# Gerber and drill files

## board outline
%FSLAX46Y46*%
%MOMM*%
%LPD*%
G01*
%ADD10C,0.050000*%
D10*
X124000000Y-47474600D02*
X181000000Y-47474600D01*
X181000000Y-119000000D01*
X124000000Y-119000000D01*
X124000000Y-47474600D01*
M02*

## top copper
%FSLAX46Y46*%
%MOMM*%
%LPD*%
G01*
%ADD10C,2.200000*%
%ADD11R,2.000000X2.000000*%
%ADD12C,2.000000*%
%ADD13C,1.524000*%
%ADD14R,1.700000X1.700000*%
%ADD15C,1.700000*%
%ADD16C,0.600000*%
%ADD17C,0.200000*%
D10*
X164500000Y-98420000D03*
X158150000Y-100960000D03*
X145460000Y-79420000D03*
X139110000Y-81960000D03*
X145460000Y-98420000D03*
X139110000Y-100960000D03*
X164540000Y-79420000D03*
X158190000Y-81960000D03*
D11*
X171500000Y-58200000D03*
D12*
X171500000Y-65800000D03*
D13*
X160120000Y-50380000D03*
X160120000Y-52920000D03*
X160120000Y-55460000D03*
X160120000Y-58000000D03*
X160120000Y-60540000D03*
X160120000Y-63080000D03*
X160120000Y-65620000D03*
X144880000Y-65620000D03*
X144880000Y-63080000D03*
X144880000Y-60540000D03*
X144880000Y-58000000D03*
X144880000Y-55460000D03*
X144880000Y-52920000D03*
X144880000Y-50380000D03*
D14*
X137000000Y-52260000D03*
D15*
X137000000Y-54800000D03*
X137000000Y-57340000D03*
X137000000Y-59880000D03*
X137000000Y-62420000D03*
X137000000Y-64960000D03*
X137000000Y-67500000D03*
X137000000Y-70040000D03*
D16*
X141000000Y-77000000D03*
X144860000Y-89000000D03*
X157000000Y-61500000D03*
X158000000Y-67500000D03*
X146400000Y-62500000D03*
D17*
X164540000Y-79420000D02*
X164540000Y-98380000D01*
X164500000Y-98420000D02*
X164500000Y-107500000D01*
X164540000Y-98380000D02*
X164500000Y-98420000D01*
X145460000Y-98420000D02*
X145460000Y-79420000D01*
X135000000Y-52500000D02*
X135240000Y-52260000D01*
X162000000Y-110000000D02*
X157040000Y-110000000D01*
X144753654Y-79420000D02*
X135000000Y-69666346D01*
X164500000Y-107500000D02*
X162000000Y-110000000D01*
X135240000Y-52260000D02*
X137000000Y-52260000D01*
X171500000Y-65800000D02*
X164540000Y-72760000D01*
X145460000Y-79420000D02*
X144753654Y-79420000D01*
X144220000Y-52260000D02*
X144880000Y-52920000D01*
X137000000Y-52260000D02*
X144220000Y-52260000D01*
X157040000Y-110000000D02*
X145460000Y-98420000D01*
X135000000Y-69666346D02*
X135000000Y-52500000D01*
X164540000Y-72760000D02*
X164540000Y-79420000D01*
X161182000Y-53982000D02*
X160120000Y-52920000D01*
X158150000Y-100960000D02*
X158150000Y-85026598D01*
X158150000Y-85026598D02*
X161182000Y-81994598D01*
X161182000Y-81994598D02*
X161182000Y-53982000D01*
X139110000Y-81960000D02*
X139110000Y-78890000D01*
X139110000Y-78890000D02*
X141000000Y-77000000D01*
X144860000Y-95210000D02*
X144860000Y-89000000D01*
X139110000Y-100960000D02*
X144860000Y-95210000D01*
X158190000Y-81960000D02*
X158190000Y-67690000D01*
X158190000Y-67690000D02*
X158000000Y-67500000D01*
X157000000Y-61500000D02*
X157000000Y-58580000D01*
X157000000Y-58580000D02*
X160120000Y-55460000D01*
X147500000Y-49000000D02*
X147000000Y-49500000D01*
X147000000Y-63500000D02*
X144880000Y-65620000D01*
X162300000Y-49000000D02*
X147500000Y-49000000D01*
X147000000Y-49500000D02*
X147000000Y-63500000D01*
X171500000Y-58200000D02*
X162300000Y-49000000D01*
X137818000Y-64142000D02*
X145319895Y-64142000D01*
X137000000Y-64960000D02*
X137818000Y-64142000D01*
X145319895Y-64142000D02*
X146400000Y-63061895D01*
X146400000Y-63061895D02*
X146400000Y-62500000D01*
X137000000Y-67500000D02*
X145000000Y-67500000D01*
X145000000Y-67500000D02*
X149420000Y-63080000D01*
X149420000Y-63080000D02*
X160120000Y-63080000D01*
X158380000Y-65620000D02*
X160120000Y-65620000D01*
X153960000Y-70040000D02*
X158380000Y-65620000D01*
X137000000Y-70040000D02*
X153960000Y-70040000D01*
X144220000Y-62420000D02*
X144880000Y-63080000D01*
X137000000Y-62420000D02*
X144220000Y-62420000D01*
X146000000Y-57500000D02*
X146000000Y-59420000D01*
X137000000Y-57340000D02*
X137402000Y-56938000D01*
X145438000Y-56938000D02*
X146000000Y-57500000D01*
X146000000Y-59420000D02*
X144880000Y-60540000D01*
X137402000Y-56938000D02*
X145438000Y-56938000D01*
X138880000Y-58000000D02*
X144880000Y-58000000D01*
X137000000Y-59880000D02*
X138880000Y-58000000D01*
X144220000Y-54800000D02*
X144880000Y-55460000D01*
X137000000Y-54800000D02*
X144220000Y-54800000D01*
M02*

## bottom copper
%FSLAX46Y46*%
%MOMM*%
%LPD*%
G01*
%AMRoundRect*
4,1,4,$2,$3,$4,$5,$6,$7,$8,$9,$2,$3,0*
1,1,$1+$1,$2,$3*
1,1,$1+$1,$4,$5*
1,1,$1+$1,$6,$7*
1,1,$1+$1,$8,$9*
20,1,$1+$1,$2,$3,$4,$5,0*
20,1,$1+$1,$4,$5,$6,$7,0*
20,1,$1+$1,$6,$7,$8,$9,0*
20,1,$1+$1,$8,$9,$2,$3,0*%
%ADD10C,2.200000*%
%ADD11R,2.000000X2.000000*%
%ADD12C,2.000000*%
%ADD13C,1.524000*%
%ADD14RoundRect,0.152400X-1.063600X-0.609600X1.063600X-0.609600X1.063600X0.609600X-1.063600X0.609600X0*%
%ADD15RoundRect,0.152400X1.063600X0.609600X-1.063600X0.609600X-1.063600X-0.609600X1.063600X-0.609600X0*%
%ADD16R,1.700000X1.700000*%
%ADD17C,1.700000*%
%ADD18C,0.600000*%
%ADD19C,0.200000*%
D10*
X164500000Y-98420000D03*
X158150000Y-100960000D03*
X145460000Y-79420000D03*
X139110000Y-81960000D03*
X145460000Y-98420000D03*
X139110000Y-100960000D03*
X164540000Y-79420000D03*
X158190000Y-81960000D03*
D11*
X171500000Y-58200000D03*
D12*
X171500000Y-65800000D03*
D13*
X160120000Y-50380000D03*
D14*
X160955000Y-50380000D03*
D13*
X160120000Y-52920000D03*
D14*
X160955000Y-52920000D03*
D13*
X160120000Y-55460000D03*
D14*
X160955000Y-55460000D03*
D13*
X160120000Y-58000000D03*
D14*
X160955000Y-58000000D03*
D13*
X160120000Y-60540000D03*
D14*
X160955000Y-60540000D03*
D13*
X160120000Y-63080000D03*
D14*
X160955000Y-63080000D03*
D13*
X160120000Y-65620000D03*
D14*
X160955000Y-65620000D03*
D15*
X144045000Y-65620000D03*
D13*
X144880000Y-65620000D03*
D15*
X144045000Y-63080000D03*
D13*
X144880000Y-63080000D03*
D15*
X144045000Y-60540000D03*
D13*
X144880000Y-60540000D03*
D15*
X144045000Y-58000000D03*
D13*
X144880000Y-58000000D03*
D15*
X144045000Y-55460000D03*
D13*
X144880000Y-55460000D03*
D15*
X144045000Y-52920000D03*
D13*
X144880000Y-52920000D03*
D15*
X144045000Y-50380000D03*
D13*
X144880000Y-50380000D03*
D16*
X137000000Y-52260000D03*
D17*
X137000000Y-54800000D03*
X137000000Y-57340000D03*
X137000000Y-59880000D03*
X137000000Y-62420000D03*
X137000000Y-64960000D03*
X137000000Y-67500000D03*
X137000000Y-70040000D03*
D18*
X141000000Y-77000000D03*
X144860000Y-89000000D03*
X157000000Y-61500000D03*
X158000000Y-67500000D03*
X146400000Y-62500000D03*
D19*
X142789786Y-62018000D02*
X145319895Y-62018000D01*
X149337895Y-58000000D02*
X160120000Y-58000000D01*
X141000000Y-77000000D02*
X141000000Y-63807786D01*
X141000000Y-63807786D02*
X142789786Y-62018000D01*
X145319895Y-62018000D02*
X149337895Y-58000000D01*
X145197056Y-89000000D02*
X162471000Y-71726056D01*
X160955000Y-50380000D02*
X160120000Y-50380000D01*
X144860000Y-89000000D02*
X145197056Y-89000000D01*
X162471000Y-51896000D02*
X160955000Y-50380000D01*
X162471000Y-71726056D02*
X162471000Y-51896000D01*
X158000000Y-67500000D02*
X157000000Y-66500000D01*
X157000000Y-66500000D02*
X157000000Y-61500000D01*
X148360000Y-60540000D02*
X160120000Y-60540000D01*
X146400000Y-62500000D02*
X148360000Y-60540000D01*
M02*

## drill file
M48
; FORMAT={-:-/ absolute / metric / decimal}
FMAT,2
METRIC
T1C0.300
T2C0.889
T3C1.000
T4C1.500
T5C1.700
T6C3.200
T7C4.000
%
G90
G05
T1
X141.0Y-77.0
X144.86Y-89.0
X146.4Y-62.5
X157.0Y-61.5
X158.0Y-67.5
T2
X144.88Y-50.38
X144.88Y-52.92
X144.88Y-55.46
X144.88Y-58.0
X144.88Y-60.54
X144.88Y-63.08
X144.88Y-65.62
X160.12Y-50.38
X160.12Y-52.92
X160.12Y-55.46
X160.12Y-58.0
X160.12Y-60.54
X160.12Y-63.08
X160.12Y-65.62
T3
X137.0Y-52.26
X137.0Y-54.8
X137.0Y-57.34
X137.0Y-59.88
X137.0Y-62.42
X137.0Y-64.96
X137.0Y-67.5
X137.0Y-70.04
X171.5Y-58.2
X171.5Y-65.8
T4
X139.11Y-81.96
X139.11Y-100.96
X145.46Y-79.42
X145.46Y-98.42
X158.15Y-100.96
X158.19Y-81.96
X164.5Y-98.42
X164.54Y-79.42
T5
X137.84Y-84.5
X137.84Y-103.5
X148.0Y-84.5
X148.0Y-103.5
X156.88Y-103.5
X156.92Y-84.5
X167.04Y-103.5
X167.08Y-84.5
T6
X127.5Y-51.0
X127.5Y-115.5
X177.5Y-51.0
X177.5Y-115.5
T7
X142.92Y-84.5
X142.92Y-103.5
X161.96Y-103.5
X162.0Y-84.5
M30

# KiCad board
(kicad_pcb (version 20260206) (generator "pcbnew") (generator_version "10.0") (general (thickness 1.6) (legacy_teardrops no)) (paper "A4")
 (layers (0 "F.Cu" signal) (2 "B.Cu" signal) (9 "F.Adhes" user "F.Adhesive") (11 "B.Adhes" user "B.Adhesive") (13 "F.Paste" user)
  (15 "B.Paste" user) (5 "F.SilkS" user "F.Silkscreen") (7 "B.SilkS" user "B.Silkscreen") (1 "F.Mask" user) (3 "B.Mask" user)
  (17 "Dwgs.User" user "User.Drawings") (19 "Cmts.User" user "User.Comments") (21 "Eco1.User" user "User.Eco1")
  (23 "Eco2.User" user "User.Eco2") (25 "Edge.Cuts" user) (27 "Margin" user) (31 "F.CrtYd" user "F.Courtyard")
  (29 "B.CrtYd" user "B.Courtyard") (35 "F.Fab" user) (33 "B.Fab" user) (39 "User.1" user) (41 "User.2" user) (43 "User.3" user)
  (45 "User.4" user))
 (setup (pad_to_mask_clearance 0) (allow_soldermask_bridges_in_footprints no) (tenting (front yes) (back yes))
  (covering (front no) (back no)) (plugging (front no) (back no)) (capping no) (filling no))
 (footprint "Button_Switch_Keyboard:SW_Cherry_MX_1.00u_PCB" (layer "F.Cu") (at 164.5 98.42)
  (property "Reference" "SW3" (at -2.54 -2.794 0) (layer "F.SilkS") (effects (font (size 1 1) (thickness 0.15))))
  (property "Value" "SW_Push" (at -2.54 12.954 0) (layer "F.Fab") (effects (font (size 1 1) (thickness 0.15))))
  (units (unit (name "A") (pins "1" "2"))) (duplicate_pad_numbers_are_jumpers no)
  (pad "" np_thru_hole circle (at -7.62 5.08) (size 1.7 1.7) (drill 1.7) (layers "*.Cu" "*.Mask"))
  (pad "" np_thru_hole circle (at -2.54 5.08) (size 4 4) (drill 4) (layers "*.Cu" "*.Mask"))
  (pad "" np_thru_hole circle (at 2.54 5.08) (size 1.7 1.7) (drill 1.7) (layers "*.Cu" "*.Mask"))
  (pad "1" thru_hole circle (at 0 0) (size 2.2 2.2) (drill 1.5) (layers "*.Cu" "*.Mask") (remove_unused_layers no) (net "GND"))
  (pad "2" thru_hole circle (at -6.35 2.54) (size 2.2 2.2) (drill 1.5) (layers "*.Cu" "*.Mask") (remove_unused_layers no)
   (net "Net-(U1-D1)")))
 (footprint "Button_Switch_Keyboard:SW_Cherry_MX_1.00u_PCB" (layer "F.Cu") (at 145.46 79.42)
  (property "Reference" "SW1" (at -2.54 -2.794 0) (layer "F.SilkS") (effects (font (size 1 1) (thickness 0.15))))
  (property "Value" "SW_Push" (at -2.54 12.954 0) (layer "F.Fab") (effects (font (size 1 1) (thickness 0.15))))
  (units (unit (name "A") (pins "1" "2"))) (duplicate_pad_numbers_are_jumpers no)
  (pad "" np_thru_hole circle (at -7.62 5.08) (size 1.7 1.7) (drill 1.7) (layers "*.Cu" "*.Mask"))
  (pad "" np_thru_hole circle (at -2.54 5.08) (size 4 4) (drill 4) (layers "*.Cu" "*.Mask"))
  (pad "" np_thru_hole circle (at 2.54 5.08) (size 1.7 1.7) (drill 1.7) (layers "*.Cu" "*.Mask"))
  (pad "1" thru_hole circle (at 0 0) (size 2.2 2.2) (drill 1.5) (layers "*.Cu" "*.Mask") (remove_unused_layers no) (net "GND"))
  (pad "2" thru_hole circle (at -6.35 2.54) (size 2.2 2.2) (drill 1.5) (layers "*.Cu" "*.Mask") (remove_unused_layers no)
   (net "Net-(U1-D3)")))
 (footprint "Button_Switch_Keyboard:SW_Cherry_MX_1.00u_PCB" (layer "F.Cu") (at 145.46 98.42)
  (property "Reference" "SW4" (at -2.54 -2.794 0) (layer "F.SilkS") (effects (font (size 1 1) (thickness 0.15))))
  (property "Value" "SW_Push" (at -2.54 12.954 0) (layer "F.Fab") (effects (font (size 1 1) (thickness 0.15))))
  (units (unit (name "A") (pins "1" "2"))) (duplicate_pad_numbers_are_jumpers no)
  (pad "" np_thru_hole circle (at -7.62 5.08) (size 1.7 1.7) (drill 1.7) (layers "*.Cu" "*.Mask"))
  (pad "" np_thru_hole circle (at -2.54 5.08) (size 4 4) (drill 4) (layers "*.Cu" "*.Mask"))
  (pad "" np_thru_hole circle (at 2.54 5.08) (size 1.7 1.7) (drill 1.7) (layers "*.Cu" "*.Mask"))
  (pad "1" thru_hole circle (at 0 0) (size 2.2 2.2) (drill 1.5) (layers "*.Cu" "*.Mask") (remove_unused_layers no) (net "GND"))
  (pad "2" thru_hole circle (at -6.35 2.54) (size 2.2 2.2) (drill 1.5) (layers "*.Cu" "*.Mask") (remove_unused_layers no)
   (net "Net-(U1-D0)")))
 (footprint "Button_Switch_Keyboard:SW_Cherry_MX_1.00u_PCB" (layer "F.Cu") (at 164.54 79.42)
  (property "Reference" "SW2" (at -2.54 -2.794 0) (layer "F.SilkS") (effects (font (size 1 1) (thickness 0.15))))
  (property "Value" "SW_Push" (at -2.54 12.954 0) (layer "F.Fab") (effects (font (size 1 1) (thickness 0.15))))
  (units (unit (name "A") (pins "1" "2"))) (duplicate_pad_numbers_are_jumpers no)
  (pad "" np_thru_hole circle (at -7.62 5.08) (size 1.7 1.7) (drill 1.7) (layers "*.Cu" "*.Mask"))
  (pad "" np_thru_hole circle (at -2.54 5.08) (size 4 4) (drill 4) (layers "*.Cu" "*.Mask"))
  (pad "" np_thru_hole circle (at 2.54 5.08) (size 1.7 1.7) (drill 1.7) (layers "*.Cu" "*.Mask"))
  (pad "1" thru_hole circle (at 0 0) (size 2.2 2.2) (drill 1.5) (layers "*.Cu" "*.Mask") (remove_unused_layers no) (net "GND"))
  (pad "2" thru_hole circle (at -6.35 2.54) (size 2.2 2.2) (drill 1.5) (layers "*.Cu" "*.Mask") (remove_unused_layers no)
   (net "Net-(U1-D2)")))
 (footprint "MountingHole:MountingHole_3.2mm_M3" (layer "F.Cu") (at 127.5 115.5 90)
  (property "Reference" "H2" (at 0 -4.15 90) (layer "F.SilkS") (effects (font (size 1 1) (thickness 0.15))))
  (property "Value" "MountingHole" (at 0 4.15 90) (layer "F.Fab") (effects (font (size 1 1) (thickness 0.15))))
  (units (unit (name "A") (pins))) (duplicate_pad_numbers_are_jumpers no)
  (pad "" np_thru_hole circle (at 0 0 90) (size 3.2 3.2) (drill 3.2) (layers "*.Cu" "*.Mask")))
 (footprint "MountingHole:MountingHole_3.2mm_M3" (layer "F.Cu") (at 177.5 51 180)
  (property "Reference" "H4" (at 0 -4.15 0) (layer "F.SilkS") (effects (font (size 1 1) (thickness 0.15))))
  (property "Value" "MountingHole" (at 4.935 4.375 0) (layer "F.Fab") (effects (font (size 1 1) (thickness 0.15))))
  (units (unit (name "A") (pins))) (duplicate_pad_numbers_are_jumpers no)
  (pad "" np_thru_hole circle (at 0 0 180) (size 3.2 3.2) (drill 3.2) (layers "*.Cu" "*.Mask")))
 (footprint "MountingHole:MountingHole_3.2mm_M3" (layer "F.Cu") (at 127.5 51 180)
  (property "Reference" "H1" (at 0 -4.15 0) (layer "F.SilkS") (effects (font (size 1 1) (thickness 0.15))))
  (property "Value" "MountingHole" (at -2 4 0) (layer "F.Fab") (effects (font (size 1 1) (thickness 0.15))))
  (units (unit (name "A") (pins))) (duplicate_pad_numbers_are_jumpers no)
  (pad "" np_thru_hole circle (at 0 0 180) (size 3.2 3.2) (drill 3.2) (layers "*.Cu" "*.Mask")))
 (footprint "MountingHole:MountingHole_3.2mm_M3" (layer "F.Cu") (at 177.5 115.5 90)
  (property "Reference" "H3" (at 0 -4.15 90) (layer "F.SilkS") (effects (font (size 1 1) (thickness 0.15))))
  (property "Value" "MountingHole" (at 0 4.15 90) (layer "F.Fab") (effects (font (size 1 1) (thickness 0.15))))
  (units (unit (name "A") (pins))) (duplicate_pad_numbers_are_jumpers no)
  (pad "" np_thru_hole circle (at 0 0 90) (size 3.2 3.2) (drill 3.2) (layers "*.Cu" "*.Mask")))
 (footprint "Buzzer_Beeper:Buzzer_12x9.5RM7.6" (layer "B.Cu") (at 171.5 58.2 -90)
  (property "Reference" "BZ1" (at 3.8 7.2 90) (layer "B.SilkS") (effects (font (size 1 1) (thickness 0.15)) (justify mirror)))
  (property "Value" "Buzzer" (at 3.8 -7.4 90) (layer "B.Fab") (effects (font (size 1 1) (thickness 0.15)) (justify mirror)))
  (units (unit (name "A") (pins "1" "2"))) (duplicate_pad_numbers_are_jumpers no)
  (pad "1" thru_hole rect (at 0 0 270) (size 2 2) (drill 1) (layers "*.Cu" "*.Mask") (remove_unused_layers no) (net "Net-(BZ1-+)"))
  (pad "2" thru_hole circle (at 7.6 0 270) (size 2 2) (drill 1) (layers "*.Cu" "*.Mask") (remove_unused_layers no) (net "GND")))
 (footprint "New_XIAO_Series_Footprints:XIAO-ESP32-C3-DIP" (layer "B.Cu") (at 152.5 58 90)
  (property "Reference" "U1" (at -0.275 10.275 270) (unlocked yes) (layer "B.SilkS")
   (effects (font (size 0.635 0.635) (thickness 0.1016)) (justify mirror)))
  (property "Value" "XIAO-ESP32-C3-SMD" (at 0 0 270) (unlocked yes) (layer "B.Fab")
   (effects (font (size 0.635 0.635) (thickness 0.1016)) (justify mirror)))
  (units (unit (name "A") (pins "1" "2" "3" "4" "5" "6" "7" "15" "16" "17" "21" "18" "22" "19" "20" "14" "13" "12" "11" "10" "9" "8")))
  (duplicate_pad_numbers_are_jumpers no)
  (pad "1" thru_hole circle (at 7.62 7.62) (size 1.524 1.524) (drill 0.889) (layers "*.Cu" "*.Mask") (remove_unused_layers no)
   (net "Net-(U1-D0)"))
  (pad "1" smd roundrect (at 7.62 8.455) (size 2.432 1.524) (layers "B.Cu" "B.Mask") (roundrect_rratio 0.1) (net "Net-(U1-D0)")
   (thermal_bridge_angle 45))
  (pad "2" thru_hole circle (at 5.08 7.62) (size 1.524 1.524) (drill 0.889) (layers "*.Cu" "*.Mask") (remove_unused_layers no)
   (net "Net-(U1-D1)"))
  (pad "2" smd roundrect (at 5.08 8.455) (size 2.432 1.524) (layers "B.Cu" "B.Mask") (roundrect_rratio 0.1) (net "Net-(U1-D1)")
   (thermal_bridge_angle 45))
  (pad "3" thru_hole circle (at 2.54 7.62) (size 1.524 1.524) (drill 0.889) (layers "*.Cu" "*.Mask") (remove_unused_layers no)
   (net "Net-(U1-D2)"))
  (pad "3" smd roundrect (at 2.54 8.455) (size 2.432 1.524) (layers "B.Cu" "B.Mask") (roundrect_rratio 0.1) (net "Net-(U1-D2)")
   (thermal_bridge_angle 45))
  (pad "4" thru_hole circle (at 0 7.62) (size 1.524 1.524) (drill 0.889) (layers "*.Cu" "*.Mask") (remove_unused_layers no)
   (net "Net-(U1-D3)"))
  (pad "4" smd roundrect (at 0 8.455) (size 2.432 1.524) (layers "B.Cu" "B.Mask") (roundrect_rratio 0.1) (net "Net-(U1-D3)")
   (thermal_bridge_angle 45))
  (pad "5" thru_hole circle (at -2.54 7.62) (size 1.524 1.524) (drill 0.889) (layers "*.Cu" "*.Mask") (remove_unused_layers no) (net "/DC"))
  (pad "5" smd roundrect (at -2.54 8.455) (size 2.432 1.524) (layers "B.Cu" "B.Mask") (roundrect_rratio 0.1) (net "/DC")
   (thermal_bridge_angle 45))
  (pad "6" thru_hole circle (at -5.08 7.62) (size 1.524 1.524) (drill 0.889) (layers "*.Cu" "*.Mask") (remove_unused_layers no) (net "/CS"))
  (pad "6" smd roundrect (at -5.08 8.455) (size 2.432 1.524) (layers "B.Cu" "B.Mask") (roundrect_rratio 0.1) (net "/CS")
   (thermal_bridge_angle 45))
  (pad "7" thru_hole circle (at -7.62 7.62) (size 1.524 1.524) (drill 0.889) (layers "*.Cu" "*.Mask") (remove_unused_layers no) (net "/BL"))
  (pad "7" smd roundrect (at -7.62 8.455) (size 2.432 1.524) (layers "B.Cu" "B.Mask") (roundrect_rratio 0.1) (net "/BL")
   (thermal_bridge_angle 45))
  (pad "8" smd roundrect (at -7.62 -8.455 180) (size 2.432 1.524) (layers "B.Cu" "B.Mask") (roundrect_rratio 0.1) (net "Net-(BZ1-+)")
   (thermal_bridge_angle 45))
  (pad "8" thru_hole circle (at -7.62 -7.62 180) (size 1.524 1.524) (drill 0.889) (layers "*.Cu" "*.Mask") (remove_unused_layers no)
   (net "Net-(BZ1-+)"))
  (pad "9" smd roundrect (at -5.08 -8.455 180) (size 2.432 1.524) (layers "B.Cu" "B.Mask") (roundrect_rratio 0.1) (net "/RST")
   (thermal_bridge_angle 45))
  (pad "9" thru_hole circle (at -5.08 -7.62 180) (size 1.524 1.524) (drill 0.889) (layers "*.Cu" "*.Mask") (remove_unused_layers no)
   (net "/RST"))
  (pad "10" smd roundrect (at -2.54 -8.455 180) (size 2.432 1.524) (layers "B.Cu" "B.Mask") (roundrect_rratio 0.1) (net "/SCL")
   (thermal_bridge_angle 45))
  (pad "10" thru_hole circle (at -2.54 -7.62 180) (size 1.524 1.524) (drill 0.889) (layers "*.Cu" "*.Mask") (remove_unused_layers no)
   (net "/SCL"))
  (pad "11" smd roundrect (at 0 -8.455 180) (size 2.432 1.524) (layers "B.Cu" "B.Mask") (roundrect_rratio 0.1) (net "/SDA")
   (thermal_bridge_angle 45))
  (pad "11" thru_hole circle (at 0 -7.62 180) (size 1.524 1.524) (drill 0.889) (layers "*.Cu" "*.Mask") (remove_unused_layers no)
   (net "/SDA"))
  (pad "12" smd roundrect (at 2.54 -8.455 180) (size 2.432 1.524) (layers "B.Cu" "B.Mask") (roundrect_rratio 0.1) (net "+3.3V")
   (thermal_bridge_angle 45))
  (pad "12" thru_hole circle (at 2.54 -7.62 180) (size 1.524 1.524) (drill 0.889) (layers "*.Cu" "*.Mask") (remove_unused_layers no)
   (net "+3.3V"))
  (pad "13" smd roundrect (at 5.08 -8.455 180) (size 2.432 1.524) (layers "B.Cu" "B.Mask") (roundrect_rratio 0.1) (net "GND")
   (thermal_bridge_angle 45))
  (pad "13" thru_hole circle (at 5.08 -7.62 180) (size 1.524 1.524) (drill 0.889) (layers "*.Cu" "*.Mask") (remove_unused_layers no)
   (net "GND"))
  (pad "14" smd roundrect (at 7.62 -8.455 180) (size 2.432 1.524) (layers "B.Cu" "B.Mask") (roundrect_rratio 0.1)
   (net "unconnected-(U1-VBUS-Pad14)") (thermal_bridge_angle 45))
  (pad "14" thru_hole circle (at 7.62 -7.62 180) (size 1.524 1.524) (drill 0.889) (layers "*.Cu" "*.Mask") (remove_unused_layers no)
   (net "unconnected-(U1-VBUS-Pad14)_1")))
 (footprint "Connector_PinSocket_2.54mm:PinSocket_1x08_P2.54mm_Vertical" (layer "B.Cu") (at 137 52.26 180)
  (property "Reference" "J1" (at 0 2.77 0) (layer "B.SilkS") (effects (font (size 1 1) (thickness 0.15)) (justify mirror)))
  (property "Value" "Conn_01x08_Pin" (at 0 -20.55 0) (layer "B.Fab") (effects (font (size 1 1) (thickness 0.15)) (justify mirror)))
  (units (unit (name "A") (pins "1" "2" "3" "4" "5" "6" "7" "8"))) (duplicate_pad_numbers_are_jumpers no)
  (pad "1" thru_hole rect (at 0 0 180) (size 1.7 1.7) (drill 1) (layers "*.Cu" "*.Mask") (remove_unused_layers no) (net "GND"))
  (pad "2" thru_hole circle (at 0 -2.54 180) (size 1.7 1.7) (drill 1) (layers "*.Cu" "*.Mask") (remove_unused_layers no) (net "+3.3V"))
  (pad "3" thru_hole circle (at 0 -5.08 180) (size 1.7 1.7) (drill 1) (layers "*.Cu" "*.Mask") (remove_unused_layers no) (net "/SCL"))
  (pad "4" thru_hole circle (at 0 -7.62 180) (size 1.7 1.7) (drill 1) (layers "*.Cu" "*.Mask") (remove_unused_layers no) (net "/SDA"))
  (pad "5" thru_hole circle (at 0 -10.16 180) (size 1.7 1.7) (drill 1) (layers "*.Cu" "*.Mask") (remove_unused_layers no) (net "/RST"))
  (pad "6" thru_hole circle (at 0 -12.7 180) (size 1.7 1.7) (drill 1) (layers "*.Cu" "*.Mask") (remove_unused_layers no) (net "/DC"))
  (pad "7" thru_hole circle (at 0 -15.24 180) (size 1.7 1.7) (drill 1) (layers "*.Cu" "*.Mask") (remove_unused_layers no) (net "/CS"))
  (pad "8" thru_hole circle (at 0 -17.78 180) (size 1.7 1.7) (drill 1) (layers "*.Cu" "*.Mask") (remove_unused_layers no) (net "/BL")))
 (gr_rect (start 124 47.4746) (end 181 119) (stroke (width 0.05) (type default)) (fill no) (layer "Edge.Cuts"))
 (segment (start 164.54 79.42) (end 164.54 98.38) (width 0.2) (layer "F.Cu") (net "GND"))
 (segment (start 164.5 98.42) (end 164.5 107.5) (width 0.2) (layer "F.Cu") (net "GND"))
 (segment (start 164.54 98.38) (end 164.5 98.42) (width 0.2) (layer "F.Cu") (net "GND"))
 (segment (start 145.46 98.42) (end 145.46 79.42) (width 0.2) (layer "F.Cu") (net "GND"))
 (segment (start 135 52.5) (end 135.24 52.26) (width 0.2) (layer "F.Cu") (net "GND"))
 (segment (start 162 110) (end 157.04 110) (width 0.2) (layer "F.Cu") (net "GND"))
 (segment (start 144.753654 79.42) (end 135 69.666346) (width 0.2) (layer "F.Cu") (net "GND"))
 (segment (start 164.5 107.5) (end 162 110) (width 0.2) (layer "F.Cu") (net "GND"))
 (segment (start 135.24 52.26) (end 137 52.26) (width 0.2) (layer "F.Cu") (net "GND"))
 (segment (start 171.5 65.8) (end 164.54 72.76) (width 0.2) (layer "F.Cu") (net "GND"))
 (segment (start 145.46 79.42) (end 144.753654 79.42) (width 0.2) (layer "F.Cu") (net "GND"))
 (segment (start 144.22 52.26) (end 144.88 52.92) (width 0.2) (layer "F.Cu") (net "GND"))
 (segment (start 137 52.26) (end 144.22 52.26) (width 0.2) (layer "F.Cu") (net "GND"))
 (segment (start 157.04 110) (end 145.46 98.42) (width 0.2) (layer "F.Cu") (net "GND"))
 (segment (start 135 69.666346) (end 135 52.5) (width 0.2) (layer "F.Cu") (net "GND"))
 (segment (start 164.54 72.76) (end 164.54 79.42) (width 0.2) (layer "F.Cu") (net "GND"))
 (segment (start 161.182 53.982) (end 160.12 52.92) (width 0.2) (layer "F.Cu") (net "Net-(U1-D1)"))
 (segment (start 158.15 100.96) (end 158.15 85.026598) (width 0.2) (layer "F.Cu") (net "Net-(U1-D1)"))
 (segment (start 158.15 85.026598) (end 161.182 81.994598) (width 0.2) (layer "F.Cu") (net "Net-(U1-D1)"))
 (segment (start 161.182 81.994598) (end 161.182 53.982) (width 0.2) (layer "F.Cu") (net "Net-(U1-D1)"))
 (segment (start 139.11 81.96) (end 139.11 78.89) (width 0.2) (layer "F.Cu") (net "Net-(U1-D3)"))
 (segment (start 139.11 78.89) (end 141 77) (width 0.2) (layer "F.Cu") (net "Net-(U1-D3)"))
 (via (at 141 77) (size 0.6) (drill 0.3) (layers "F.Cu" "B.Cu") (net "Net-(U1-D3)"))
 (segment (start 142.789786 62.018) (end 145.319895 62.018) (width 0.2) (layer "B.Cu") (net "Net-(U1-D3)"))
 (segment (start 149.337895 58) (end 160.12 58) (width 0.2) (layer "B.Cu") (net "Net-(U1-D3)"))
 (segment (start 141 77) (end 141 63.807786) (width 0.2) (layer "B.Cu") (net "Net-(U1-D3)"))
 (segment (start 141 63.807786) (end 142.789786 62.018) (width 0.2) (layer "B.Cu") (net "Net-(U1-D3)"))
 (segment (start 145.319895 62.018) (end 149.337895 58) (width 0.2) (layer "B.Cu") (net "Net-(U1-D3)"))
 (segment (start 144.86 95.21) (end 144.86 89) (width 0.2) (layer "F.Cu") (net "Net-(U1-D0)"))
 (segment (start 139.11 100.96) (end 144.86 95.21) (width 0.2) (layer "F.Cu") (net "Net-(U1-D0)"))
 (via (at 144.86 89) (size 0.6) (drill 0.3) (layers "F.Cu" "B.Cu") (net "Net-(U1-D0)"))
 (segment (start 145.197056 89) (end 162.471 71.726056) (width 0.2) (layer "B.Cu") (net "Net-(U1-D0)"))
 (segment (start 160.955 50.38) (end 160.12 50.38) (width 0.2) (layer "B.Cu") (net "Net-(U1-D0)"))
 (segment (start 144.86 89) (end 145.197056 89) (width 0.2) (layer "B.Cu") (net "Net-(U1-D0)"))
 (segment (start 162.471 51.896) (end 160.955 50.38) (width 0.2) (layer "B.Cu") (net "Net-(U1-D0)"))
 (segment (start 162.471 71.726056) (end 162.471 51.896) (width 0.2) (layer "B.Cu") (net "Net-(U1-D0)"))
 (segment (start 158.19 81.96) (end 158.19 67.69) (width 0.2) (layer "F.Cu") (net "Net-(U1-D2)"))
 (segment (start 158.19 67.69) (end 158 67.5) (width 0.2) (layer "F.Cu") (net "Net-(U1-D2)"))
 (segment (start 157 61.5) (end 157 58.58) (width 0.2) (layer "F.Cu") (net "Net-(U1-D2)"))
 (segment (start 157 58.58) (end 160.12 55.46) (width 0.2) (layer "F.Cu") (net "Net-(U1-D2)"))
 (via (at 157 61.5) (size 0.6) (drill 0.3) (layers "F.Cu" "B.Cu") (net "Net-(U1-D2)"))
 (via (at 158 67.5) (size 0.6) (drill 0.3) (layers "F.Cu" "B.Cu") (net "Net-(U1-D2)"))
 (segment (start 158 67.5) (end 157 66.5) (width 0.2) (layer "B.Cu") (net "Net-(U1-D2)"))
 (segment (start 157 66.5) (end 157 61.5) (width 0.2) (layer "B.Cu") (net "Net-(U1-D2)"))
 (segment (start 147.5 49) (end 147 49.5) (width 0.2) (layer "F.Cu") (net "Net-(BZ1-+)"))
 (segment (start 147 63.5) (end 144.88 65.62) (width 0.2) (layer "F.Cu") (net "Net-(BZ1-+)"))
 (segment (start 162.3 49) (end 147.5 49) (width 0.2) (layer "F.Cu") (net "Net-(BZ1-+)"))
 (segment (start 147 49.5) (end 147 63.5) (width 0.2) (layer "F.Cu") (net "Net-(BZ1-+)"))
 (segment (start 171.5 58.2) (end 162.3 49) (width 0.2) (layer "F.Cu") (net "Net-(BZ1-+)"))
 (segment (start 137.818 64.142) (end 145.319895 64.142) (width 0.2) (layer "F.Cu") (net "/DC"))
 (segment (start 137 64.96) (end 137.818 64.142) (width 0.2) (layer "F.Cu") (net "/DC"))
 (segment (start 145.319895 64.142) (end 146.4 63.061895) (width 0.2) (layer "F.Cu") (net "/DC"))
 (segment (start 146.4 63.061895) (end 146.4 62.5) (width 0.2) (layer "F.Cu") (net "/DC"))
 (via (at 146.4 62.5) (size 0.6) (drill 0.3) (layers "F.Cu" "B.Cu") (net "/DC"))
 (segment (start 148.36 60.54) (end 160.12 60.54) (width 0.2) (layer "B.Cu") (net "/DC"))
 (segment (start 146.4 62.5) (end 148.36 60.54) (width 0.2) (layer "B.Cu") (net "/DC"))
 (segment (start 137 67.5) (end 145 67.5) (width 0.2) (layer "F.Cu") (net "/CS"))
 (segment (start 145 67.5) (end 149.42 63.08) (width 0.2) (layer "F.Cu") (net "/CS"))
 (segment (start 149.42 63.08) (end 160.12 63.08) (width 0.2) (layer "F.Cu") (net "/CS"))
 (segment (start 158.38 65.62) (end 160.12 65.62) (width 0.2) (layer "F.Cu") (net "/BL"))
 (segment (start 153.96 70.04) (end 158.38 65.62) (width 0.2) (layer "F.Cu") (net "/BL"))
 (segment (start 137 70.04) (end 153.96 70.04) (width 0.2) (layer "F.Cu") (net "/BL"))
 (segment (start 144.22 62.42) (end 144.88 63.08) (width 0.2) (layer "F.Cu") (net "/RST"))
 (segment (start 137 62.42) (end 144.22 62.42) (width 0.2) (layer "F.Cu") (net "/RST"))
 (segment (start 146 57.5) (end 146 59.42) (width 0.2) (layer "F.Cu") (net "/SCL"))
 (segment (start 137 57.34) (end 137.402 56.938) (width 0.2) (layer "F.Cu") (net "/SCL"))
 (segment (start 145.438 56.938) (end 146 57.5) (width 0.2) (layer "F.Cu") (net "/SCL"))
 (segment (start 146 59.42) (end 144.88 60.54) (width 0.2) (layer "F.Cu") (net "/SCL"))
 (segment (start 137.402 56.938) (end 145.438 56.938) (width 0.2) (layer "F.Cu") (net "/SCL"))
 (segment (start 138.88 58) (end 144.88 58) (width 0.2) (layer "F.Cu") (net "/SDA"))
 (segment (start 137 59.88) (end 138.88 58) (width 0.2) (layer "F.Cu") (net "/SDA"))
 (segment (start 144.22 54.8) (end 144.88 55.46) (width 0.2) (layer "F.Cu") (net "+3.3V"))
 (segment (start 137 54.8) (end 144.22 54.8) (width 0.2) (layer "F.Cu") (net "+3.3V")))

